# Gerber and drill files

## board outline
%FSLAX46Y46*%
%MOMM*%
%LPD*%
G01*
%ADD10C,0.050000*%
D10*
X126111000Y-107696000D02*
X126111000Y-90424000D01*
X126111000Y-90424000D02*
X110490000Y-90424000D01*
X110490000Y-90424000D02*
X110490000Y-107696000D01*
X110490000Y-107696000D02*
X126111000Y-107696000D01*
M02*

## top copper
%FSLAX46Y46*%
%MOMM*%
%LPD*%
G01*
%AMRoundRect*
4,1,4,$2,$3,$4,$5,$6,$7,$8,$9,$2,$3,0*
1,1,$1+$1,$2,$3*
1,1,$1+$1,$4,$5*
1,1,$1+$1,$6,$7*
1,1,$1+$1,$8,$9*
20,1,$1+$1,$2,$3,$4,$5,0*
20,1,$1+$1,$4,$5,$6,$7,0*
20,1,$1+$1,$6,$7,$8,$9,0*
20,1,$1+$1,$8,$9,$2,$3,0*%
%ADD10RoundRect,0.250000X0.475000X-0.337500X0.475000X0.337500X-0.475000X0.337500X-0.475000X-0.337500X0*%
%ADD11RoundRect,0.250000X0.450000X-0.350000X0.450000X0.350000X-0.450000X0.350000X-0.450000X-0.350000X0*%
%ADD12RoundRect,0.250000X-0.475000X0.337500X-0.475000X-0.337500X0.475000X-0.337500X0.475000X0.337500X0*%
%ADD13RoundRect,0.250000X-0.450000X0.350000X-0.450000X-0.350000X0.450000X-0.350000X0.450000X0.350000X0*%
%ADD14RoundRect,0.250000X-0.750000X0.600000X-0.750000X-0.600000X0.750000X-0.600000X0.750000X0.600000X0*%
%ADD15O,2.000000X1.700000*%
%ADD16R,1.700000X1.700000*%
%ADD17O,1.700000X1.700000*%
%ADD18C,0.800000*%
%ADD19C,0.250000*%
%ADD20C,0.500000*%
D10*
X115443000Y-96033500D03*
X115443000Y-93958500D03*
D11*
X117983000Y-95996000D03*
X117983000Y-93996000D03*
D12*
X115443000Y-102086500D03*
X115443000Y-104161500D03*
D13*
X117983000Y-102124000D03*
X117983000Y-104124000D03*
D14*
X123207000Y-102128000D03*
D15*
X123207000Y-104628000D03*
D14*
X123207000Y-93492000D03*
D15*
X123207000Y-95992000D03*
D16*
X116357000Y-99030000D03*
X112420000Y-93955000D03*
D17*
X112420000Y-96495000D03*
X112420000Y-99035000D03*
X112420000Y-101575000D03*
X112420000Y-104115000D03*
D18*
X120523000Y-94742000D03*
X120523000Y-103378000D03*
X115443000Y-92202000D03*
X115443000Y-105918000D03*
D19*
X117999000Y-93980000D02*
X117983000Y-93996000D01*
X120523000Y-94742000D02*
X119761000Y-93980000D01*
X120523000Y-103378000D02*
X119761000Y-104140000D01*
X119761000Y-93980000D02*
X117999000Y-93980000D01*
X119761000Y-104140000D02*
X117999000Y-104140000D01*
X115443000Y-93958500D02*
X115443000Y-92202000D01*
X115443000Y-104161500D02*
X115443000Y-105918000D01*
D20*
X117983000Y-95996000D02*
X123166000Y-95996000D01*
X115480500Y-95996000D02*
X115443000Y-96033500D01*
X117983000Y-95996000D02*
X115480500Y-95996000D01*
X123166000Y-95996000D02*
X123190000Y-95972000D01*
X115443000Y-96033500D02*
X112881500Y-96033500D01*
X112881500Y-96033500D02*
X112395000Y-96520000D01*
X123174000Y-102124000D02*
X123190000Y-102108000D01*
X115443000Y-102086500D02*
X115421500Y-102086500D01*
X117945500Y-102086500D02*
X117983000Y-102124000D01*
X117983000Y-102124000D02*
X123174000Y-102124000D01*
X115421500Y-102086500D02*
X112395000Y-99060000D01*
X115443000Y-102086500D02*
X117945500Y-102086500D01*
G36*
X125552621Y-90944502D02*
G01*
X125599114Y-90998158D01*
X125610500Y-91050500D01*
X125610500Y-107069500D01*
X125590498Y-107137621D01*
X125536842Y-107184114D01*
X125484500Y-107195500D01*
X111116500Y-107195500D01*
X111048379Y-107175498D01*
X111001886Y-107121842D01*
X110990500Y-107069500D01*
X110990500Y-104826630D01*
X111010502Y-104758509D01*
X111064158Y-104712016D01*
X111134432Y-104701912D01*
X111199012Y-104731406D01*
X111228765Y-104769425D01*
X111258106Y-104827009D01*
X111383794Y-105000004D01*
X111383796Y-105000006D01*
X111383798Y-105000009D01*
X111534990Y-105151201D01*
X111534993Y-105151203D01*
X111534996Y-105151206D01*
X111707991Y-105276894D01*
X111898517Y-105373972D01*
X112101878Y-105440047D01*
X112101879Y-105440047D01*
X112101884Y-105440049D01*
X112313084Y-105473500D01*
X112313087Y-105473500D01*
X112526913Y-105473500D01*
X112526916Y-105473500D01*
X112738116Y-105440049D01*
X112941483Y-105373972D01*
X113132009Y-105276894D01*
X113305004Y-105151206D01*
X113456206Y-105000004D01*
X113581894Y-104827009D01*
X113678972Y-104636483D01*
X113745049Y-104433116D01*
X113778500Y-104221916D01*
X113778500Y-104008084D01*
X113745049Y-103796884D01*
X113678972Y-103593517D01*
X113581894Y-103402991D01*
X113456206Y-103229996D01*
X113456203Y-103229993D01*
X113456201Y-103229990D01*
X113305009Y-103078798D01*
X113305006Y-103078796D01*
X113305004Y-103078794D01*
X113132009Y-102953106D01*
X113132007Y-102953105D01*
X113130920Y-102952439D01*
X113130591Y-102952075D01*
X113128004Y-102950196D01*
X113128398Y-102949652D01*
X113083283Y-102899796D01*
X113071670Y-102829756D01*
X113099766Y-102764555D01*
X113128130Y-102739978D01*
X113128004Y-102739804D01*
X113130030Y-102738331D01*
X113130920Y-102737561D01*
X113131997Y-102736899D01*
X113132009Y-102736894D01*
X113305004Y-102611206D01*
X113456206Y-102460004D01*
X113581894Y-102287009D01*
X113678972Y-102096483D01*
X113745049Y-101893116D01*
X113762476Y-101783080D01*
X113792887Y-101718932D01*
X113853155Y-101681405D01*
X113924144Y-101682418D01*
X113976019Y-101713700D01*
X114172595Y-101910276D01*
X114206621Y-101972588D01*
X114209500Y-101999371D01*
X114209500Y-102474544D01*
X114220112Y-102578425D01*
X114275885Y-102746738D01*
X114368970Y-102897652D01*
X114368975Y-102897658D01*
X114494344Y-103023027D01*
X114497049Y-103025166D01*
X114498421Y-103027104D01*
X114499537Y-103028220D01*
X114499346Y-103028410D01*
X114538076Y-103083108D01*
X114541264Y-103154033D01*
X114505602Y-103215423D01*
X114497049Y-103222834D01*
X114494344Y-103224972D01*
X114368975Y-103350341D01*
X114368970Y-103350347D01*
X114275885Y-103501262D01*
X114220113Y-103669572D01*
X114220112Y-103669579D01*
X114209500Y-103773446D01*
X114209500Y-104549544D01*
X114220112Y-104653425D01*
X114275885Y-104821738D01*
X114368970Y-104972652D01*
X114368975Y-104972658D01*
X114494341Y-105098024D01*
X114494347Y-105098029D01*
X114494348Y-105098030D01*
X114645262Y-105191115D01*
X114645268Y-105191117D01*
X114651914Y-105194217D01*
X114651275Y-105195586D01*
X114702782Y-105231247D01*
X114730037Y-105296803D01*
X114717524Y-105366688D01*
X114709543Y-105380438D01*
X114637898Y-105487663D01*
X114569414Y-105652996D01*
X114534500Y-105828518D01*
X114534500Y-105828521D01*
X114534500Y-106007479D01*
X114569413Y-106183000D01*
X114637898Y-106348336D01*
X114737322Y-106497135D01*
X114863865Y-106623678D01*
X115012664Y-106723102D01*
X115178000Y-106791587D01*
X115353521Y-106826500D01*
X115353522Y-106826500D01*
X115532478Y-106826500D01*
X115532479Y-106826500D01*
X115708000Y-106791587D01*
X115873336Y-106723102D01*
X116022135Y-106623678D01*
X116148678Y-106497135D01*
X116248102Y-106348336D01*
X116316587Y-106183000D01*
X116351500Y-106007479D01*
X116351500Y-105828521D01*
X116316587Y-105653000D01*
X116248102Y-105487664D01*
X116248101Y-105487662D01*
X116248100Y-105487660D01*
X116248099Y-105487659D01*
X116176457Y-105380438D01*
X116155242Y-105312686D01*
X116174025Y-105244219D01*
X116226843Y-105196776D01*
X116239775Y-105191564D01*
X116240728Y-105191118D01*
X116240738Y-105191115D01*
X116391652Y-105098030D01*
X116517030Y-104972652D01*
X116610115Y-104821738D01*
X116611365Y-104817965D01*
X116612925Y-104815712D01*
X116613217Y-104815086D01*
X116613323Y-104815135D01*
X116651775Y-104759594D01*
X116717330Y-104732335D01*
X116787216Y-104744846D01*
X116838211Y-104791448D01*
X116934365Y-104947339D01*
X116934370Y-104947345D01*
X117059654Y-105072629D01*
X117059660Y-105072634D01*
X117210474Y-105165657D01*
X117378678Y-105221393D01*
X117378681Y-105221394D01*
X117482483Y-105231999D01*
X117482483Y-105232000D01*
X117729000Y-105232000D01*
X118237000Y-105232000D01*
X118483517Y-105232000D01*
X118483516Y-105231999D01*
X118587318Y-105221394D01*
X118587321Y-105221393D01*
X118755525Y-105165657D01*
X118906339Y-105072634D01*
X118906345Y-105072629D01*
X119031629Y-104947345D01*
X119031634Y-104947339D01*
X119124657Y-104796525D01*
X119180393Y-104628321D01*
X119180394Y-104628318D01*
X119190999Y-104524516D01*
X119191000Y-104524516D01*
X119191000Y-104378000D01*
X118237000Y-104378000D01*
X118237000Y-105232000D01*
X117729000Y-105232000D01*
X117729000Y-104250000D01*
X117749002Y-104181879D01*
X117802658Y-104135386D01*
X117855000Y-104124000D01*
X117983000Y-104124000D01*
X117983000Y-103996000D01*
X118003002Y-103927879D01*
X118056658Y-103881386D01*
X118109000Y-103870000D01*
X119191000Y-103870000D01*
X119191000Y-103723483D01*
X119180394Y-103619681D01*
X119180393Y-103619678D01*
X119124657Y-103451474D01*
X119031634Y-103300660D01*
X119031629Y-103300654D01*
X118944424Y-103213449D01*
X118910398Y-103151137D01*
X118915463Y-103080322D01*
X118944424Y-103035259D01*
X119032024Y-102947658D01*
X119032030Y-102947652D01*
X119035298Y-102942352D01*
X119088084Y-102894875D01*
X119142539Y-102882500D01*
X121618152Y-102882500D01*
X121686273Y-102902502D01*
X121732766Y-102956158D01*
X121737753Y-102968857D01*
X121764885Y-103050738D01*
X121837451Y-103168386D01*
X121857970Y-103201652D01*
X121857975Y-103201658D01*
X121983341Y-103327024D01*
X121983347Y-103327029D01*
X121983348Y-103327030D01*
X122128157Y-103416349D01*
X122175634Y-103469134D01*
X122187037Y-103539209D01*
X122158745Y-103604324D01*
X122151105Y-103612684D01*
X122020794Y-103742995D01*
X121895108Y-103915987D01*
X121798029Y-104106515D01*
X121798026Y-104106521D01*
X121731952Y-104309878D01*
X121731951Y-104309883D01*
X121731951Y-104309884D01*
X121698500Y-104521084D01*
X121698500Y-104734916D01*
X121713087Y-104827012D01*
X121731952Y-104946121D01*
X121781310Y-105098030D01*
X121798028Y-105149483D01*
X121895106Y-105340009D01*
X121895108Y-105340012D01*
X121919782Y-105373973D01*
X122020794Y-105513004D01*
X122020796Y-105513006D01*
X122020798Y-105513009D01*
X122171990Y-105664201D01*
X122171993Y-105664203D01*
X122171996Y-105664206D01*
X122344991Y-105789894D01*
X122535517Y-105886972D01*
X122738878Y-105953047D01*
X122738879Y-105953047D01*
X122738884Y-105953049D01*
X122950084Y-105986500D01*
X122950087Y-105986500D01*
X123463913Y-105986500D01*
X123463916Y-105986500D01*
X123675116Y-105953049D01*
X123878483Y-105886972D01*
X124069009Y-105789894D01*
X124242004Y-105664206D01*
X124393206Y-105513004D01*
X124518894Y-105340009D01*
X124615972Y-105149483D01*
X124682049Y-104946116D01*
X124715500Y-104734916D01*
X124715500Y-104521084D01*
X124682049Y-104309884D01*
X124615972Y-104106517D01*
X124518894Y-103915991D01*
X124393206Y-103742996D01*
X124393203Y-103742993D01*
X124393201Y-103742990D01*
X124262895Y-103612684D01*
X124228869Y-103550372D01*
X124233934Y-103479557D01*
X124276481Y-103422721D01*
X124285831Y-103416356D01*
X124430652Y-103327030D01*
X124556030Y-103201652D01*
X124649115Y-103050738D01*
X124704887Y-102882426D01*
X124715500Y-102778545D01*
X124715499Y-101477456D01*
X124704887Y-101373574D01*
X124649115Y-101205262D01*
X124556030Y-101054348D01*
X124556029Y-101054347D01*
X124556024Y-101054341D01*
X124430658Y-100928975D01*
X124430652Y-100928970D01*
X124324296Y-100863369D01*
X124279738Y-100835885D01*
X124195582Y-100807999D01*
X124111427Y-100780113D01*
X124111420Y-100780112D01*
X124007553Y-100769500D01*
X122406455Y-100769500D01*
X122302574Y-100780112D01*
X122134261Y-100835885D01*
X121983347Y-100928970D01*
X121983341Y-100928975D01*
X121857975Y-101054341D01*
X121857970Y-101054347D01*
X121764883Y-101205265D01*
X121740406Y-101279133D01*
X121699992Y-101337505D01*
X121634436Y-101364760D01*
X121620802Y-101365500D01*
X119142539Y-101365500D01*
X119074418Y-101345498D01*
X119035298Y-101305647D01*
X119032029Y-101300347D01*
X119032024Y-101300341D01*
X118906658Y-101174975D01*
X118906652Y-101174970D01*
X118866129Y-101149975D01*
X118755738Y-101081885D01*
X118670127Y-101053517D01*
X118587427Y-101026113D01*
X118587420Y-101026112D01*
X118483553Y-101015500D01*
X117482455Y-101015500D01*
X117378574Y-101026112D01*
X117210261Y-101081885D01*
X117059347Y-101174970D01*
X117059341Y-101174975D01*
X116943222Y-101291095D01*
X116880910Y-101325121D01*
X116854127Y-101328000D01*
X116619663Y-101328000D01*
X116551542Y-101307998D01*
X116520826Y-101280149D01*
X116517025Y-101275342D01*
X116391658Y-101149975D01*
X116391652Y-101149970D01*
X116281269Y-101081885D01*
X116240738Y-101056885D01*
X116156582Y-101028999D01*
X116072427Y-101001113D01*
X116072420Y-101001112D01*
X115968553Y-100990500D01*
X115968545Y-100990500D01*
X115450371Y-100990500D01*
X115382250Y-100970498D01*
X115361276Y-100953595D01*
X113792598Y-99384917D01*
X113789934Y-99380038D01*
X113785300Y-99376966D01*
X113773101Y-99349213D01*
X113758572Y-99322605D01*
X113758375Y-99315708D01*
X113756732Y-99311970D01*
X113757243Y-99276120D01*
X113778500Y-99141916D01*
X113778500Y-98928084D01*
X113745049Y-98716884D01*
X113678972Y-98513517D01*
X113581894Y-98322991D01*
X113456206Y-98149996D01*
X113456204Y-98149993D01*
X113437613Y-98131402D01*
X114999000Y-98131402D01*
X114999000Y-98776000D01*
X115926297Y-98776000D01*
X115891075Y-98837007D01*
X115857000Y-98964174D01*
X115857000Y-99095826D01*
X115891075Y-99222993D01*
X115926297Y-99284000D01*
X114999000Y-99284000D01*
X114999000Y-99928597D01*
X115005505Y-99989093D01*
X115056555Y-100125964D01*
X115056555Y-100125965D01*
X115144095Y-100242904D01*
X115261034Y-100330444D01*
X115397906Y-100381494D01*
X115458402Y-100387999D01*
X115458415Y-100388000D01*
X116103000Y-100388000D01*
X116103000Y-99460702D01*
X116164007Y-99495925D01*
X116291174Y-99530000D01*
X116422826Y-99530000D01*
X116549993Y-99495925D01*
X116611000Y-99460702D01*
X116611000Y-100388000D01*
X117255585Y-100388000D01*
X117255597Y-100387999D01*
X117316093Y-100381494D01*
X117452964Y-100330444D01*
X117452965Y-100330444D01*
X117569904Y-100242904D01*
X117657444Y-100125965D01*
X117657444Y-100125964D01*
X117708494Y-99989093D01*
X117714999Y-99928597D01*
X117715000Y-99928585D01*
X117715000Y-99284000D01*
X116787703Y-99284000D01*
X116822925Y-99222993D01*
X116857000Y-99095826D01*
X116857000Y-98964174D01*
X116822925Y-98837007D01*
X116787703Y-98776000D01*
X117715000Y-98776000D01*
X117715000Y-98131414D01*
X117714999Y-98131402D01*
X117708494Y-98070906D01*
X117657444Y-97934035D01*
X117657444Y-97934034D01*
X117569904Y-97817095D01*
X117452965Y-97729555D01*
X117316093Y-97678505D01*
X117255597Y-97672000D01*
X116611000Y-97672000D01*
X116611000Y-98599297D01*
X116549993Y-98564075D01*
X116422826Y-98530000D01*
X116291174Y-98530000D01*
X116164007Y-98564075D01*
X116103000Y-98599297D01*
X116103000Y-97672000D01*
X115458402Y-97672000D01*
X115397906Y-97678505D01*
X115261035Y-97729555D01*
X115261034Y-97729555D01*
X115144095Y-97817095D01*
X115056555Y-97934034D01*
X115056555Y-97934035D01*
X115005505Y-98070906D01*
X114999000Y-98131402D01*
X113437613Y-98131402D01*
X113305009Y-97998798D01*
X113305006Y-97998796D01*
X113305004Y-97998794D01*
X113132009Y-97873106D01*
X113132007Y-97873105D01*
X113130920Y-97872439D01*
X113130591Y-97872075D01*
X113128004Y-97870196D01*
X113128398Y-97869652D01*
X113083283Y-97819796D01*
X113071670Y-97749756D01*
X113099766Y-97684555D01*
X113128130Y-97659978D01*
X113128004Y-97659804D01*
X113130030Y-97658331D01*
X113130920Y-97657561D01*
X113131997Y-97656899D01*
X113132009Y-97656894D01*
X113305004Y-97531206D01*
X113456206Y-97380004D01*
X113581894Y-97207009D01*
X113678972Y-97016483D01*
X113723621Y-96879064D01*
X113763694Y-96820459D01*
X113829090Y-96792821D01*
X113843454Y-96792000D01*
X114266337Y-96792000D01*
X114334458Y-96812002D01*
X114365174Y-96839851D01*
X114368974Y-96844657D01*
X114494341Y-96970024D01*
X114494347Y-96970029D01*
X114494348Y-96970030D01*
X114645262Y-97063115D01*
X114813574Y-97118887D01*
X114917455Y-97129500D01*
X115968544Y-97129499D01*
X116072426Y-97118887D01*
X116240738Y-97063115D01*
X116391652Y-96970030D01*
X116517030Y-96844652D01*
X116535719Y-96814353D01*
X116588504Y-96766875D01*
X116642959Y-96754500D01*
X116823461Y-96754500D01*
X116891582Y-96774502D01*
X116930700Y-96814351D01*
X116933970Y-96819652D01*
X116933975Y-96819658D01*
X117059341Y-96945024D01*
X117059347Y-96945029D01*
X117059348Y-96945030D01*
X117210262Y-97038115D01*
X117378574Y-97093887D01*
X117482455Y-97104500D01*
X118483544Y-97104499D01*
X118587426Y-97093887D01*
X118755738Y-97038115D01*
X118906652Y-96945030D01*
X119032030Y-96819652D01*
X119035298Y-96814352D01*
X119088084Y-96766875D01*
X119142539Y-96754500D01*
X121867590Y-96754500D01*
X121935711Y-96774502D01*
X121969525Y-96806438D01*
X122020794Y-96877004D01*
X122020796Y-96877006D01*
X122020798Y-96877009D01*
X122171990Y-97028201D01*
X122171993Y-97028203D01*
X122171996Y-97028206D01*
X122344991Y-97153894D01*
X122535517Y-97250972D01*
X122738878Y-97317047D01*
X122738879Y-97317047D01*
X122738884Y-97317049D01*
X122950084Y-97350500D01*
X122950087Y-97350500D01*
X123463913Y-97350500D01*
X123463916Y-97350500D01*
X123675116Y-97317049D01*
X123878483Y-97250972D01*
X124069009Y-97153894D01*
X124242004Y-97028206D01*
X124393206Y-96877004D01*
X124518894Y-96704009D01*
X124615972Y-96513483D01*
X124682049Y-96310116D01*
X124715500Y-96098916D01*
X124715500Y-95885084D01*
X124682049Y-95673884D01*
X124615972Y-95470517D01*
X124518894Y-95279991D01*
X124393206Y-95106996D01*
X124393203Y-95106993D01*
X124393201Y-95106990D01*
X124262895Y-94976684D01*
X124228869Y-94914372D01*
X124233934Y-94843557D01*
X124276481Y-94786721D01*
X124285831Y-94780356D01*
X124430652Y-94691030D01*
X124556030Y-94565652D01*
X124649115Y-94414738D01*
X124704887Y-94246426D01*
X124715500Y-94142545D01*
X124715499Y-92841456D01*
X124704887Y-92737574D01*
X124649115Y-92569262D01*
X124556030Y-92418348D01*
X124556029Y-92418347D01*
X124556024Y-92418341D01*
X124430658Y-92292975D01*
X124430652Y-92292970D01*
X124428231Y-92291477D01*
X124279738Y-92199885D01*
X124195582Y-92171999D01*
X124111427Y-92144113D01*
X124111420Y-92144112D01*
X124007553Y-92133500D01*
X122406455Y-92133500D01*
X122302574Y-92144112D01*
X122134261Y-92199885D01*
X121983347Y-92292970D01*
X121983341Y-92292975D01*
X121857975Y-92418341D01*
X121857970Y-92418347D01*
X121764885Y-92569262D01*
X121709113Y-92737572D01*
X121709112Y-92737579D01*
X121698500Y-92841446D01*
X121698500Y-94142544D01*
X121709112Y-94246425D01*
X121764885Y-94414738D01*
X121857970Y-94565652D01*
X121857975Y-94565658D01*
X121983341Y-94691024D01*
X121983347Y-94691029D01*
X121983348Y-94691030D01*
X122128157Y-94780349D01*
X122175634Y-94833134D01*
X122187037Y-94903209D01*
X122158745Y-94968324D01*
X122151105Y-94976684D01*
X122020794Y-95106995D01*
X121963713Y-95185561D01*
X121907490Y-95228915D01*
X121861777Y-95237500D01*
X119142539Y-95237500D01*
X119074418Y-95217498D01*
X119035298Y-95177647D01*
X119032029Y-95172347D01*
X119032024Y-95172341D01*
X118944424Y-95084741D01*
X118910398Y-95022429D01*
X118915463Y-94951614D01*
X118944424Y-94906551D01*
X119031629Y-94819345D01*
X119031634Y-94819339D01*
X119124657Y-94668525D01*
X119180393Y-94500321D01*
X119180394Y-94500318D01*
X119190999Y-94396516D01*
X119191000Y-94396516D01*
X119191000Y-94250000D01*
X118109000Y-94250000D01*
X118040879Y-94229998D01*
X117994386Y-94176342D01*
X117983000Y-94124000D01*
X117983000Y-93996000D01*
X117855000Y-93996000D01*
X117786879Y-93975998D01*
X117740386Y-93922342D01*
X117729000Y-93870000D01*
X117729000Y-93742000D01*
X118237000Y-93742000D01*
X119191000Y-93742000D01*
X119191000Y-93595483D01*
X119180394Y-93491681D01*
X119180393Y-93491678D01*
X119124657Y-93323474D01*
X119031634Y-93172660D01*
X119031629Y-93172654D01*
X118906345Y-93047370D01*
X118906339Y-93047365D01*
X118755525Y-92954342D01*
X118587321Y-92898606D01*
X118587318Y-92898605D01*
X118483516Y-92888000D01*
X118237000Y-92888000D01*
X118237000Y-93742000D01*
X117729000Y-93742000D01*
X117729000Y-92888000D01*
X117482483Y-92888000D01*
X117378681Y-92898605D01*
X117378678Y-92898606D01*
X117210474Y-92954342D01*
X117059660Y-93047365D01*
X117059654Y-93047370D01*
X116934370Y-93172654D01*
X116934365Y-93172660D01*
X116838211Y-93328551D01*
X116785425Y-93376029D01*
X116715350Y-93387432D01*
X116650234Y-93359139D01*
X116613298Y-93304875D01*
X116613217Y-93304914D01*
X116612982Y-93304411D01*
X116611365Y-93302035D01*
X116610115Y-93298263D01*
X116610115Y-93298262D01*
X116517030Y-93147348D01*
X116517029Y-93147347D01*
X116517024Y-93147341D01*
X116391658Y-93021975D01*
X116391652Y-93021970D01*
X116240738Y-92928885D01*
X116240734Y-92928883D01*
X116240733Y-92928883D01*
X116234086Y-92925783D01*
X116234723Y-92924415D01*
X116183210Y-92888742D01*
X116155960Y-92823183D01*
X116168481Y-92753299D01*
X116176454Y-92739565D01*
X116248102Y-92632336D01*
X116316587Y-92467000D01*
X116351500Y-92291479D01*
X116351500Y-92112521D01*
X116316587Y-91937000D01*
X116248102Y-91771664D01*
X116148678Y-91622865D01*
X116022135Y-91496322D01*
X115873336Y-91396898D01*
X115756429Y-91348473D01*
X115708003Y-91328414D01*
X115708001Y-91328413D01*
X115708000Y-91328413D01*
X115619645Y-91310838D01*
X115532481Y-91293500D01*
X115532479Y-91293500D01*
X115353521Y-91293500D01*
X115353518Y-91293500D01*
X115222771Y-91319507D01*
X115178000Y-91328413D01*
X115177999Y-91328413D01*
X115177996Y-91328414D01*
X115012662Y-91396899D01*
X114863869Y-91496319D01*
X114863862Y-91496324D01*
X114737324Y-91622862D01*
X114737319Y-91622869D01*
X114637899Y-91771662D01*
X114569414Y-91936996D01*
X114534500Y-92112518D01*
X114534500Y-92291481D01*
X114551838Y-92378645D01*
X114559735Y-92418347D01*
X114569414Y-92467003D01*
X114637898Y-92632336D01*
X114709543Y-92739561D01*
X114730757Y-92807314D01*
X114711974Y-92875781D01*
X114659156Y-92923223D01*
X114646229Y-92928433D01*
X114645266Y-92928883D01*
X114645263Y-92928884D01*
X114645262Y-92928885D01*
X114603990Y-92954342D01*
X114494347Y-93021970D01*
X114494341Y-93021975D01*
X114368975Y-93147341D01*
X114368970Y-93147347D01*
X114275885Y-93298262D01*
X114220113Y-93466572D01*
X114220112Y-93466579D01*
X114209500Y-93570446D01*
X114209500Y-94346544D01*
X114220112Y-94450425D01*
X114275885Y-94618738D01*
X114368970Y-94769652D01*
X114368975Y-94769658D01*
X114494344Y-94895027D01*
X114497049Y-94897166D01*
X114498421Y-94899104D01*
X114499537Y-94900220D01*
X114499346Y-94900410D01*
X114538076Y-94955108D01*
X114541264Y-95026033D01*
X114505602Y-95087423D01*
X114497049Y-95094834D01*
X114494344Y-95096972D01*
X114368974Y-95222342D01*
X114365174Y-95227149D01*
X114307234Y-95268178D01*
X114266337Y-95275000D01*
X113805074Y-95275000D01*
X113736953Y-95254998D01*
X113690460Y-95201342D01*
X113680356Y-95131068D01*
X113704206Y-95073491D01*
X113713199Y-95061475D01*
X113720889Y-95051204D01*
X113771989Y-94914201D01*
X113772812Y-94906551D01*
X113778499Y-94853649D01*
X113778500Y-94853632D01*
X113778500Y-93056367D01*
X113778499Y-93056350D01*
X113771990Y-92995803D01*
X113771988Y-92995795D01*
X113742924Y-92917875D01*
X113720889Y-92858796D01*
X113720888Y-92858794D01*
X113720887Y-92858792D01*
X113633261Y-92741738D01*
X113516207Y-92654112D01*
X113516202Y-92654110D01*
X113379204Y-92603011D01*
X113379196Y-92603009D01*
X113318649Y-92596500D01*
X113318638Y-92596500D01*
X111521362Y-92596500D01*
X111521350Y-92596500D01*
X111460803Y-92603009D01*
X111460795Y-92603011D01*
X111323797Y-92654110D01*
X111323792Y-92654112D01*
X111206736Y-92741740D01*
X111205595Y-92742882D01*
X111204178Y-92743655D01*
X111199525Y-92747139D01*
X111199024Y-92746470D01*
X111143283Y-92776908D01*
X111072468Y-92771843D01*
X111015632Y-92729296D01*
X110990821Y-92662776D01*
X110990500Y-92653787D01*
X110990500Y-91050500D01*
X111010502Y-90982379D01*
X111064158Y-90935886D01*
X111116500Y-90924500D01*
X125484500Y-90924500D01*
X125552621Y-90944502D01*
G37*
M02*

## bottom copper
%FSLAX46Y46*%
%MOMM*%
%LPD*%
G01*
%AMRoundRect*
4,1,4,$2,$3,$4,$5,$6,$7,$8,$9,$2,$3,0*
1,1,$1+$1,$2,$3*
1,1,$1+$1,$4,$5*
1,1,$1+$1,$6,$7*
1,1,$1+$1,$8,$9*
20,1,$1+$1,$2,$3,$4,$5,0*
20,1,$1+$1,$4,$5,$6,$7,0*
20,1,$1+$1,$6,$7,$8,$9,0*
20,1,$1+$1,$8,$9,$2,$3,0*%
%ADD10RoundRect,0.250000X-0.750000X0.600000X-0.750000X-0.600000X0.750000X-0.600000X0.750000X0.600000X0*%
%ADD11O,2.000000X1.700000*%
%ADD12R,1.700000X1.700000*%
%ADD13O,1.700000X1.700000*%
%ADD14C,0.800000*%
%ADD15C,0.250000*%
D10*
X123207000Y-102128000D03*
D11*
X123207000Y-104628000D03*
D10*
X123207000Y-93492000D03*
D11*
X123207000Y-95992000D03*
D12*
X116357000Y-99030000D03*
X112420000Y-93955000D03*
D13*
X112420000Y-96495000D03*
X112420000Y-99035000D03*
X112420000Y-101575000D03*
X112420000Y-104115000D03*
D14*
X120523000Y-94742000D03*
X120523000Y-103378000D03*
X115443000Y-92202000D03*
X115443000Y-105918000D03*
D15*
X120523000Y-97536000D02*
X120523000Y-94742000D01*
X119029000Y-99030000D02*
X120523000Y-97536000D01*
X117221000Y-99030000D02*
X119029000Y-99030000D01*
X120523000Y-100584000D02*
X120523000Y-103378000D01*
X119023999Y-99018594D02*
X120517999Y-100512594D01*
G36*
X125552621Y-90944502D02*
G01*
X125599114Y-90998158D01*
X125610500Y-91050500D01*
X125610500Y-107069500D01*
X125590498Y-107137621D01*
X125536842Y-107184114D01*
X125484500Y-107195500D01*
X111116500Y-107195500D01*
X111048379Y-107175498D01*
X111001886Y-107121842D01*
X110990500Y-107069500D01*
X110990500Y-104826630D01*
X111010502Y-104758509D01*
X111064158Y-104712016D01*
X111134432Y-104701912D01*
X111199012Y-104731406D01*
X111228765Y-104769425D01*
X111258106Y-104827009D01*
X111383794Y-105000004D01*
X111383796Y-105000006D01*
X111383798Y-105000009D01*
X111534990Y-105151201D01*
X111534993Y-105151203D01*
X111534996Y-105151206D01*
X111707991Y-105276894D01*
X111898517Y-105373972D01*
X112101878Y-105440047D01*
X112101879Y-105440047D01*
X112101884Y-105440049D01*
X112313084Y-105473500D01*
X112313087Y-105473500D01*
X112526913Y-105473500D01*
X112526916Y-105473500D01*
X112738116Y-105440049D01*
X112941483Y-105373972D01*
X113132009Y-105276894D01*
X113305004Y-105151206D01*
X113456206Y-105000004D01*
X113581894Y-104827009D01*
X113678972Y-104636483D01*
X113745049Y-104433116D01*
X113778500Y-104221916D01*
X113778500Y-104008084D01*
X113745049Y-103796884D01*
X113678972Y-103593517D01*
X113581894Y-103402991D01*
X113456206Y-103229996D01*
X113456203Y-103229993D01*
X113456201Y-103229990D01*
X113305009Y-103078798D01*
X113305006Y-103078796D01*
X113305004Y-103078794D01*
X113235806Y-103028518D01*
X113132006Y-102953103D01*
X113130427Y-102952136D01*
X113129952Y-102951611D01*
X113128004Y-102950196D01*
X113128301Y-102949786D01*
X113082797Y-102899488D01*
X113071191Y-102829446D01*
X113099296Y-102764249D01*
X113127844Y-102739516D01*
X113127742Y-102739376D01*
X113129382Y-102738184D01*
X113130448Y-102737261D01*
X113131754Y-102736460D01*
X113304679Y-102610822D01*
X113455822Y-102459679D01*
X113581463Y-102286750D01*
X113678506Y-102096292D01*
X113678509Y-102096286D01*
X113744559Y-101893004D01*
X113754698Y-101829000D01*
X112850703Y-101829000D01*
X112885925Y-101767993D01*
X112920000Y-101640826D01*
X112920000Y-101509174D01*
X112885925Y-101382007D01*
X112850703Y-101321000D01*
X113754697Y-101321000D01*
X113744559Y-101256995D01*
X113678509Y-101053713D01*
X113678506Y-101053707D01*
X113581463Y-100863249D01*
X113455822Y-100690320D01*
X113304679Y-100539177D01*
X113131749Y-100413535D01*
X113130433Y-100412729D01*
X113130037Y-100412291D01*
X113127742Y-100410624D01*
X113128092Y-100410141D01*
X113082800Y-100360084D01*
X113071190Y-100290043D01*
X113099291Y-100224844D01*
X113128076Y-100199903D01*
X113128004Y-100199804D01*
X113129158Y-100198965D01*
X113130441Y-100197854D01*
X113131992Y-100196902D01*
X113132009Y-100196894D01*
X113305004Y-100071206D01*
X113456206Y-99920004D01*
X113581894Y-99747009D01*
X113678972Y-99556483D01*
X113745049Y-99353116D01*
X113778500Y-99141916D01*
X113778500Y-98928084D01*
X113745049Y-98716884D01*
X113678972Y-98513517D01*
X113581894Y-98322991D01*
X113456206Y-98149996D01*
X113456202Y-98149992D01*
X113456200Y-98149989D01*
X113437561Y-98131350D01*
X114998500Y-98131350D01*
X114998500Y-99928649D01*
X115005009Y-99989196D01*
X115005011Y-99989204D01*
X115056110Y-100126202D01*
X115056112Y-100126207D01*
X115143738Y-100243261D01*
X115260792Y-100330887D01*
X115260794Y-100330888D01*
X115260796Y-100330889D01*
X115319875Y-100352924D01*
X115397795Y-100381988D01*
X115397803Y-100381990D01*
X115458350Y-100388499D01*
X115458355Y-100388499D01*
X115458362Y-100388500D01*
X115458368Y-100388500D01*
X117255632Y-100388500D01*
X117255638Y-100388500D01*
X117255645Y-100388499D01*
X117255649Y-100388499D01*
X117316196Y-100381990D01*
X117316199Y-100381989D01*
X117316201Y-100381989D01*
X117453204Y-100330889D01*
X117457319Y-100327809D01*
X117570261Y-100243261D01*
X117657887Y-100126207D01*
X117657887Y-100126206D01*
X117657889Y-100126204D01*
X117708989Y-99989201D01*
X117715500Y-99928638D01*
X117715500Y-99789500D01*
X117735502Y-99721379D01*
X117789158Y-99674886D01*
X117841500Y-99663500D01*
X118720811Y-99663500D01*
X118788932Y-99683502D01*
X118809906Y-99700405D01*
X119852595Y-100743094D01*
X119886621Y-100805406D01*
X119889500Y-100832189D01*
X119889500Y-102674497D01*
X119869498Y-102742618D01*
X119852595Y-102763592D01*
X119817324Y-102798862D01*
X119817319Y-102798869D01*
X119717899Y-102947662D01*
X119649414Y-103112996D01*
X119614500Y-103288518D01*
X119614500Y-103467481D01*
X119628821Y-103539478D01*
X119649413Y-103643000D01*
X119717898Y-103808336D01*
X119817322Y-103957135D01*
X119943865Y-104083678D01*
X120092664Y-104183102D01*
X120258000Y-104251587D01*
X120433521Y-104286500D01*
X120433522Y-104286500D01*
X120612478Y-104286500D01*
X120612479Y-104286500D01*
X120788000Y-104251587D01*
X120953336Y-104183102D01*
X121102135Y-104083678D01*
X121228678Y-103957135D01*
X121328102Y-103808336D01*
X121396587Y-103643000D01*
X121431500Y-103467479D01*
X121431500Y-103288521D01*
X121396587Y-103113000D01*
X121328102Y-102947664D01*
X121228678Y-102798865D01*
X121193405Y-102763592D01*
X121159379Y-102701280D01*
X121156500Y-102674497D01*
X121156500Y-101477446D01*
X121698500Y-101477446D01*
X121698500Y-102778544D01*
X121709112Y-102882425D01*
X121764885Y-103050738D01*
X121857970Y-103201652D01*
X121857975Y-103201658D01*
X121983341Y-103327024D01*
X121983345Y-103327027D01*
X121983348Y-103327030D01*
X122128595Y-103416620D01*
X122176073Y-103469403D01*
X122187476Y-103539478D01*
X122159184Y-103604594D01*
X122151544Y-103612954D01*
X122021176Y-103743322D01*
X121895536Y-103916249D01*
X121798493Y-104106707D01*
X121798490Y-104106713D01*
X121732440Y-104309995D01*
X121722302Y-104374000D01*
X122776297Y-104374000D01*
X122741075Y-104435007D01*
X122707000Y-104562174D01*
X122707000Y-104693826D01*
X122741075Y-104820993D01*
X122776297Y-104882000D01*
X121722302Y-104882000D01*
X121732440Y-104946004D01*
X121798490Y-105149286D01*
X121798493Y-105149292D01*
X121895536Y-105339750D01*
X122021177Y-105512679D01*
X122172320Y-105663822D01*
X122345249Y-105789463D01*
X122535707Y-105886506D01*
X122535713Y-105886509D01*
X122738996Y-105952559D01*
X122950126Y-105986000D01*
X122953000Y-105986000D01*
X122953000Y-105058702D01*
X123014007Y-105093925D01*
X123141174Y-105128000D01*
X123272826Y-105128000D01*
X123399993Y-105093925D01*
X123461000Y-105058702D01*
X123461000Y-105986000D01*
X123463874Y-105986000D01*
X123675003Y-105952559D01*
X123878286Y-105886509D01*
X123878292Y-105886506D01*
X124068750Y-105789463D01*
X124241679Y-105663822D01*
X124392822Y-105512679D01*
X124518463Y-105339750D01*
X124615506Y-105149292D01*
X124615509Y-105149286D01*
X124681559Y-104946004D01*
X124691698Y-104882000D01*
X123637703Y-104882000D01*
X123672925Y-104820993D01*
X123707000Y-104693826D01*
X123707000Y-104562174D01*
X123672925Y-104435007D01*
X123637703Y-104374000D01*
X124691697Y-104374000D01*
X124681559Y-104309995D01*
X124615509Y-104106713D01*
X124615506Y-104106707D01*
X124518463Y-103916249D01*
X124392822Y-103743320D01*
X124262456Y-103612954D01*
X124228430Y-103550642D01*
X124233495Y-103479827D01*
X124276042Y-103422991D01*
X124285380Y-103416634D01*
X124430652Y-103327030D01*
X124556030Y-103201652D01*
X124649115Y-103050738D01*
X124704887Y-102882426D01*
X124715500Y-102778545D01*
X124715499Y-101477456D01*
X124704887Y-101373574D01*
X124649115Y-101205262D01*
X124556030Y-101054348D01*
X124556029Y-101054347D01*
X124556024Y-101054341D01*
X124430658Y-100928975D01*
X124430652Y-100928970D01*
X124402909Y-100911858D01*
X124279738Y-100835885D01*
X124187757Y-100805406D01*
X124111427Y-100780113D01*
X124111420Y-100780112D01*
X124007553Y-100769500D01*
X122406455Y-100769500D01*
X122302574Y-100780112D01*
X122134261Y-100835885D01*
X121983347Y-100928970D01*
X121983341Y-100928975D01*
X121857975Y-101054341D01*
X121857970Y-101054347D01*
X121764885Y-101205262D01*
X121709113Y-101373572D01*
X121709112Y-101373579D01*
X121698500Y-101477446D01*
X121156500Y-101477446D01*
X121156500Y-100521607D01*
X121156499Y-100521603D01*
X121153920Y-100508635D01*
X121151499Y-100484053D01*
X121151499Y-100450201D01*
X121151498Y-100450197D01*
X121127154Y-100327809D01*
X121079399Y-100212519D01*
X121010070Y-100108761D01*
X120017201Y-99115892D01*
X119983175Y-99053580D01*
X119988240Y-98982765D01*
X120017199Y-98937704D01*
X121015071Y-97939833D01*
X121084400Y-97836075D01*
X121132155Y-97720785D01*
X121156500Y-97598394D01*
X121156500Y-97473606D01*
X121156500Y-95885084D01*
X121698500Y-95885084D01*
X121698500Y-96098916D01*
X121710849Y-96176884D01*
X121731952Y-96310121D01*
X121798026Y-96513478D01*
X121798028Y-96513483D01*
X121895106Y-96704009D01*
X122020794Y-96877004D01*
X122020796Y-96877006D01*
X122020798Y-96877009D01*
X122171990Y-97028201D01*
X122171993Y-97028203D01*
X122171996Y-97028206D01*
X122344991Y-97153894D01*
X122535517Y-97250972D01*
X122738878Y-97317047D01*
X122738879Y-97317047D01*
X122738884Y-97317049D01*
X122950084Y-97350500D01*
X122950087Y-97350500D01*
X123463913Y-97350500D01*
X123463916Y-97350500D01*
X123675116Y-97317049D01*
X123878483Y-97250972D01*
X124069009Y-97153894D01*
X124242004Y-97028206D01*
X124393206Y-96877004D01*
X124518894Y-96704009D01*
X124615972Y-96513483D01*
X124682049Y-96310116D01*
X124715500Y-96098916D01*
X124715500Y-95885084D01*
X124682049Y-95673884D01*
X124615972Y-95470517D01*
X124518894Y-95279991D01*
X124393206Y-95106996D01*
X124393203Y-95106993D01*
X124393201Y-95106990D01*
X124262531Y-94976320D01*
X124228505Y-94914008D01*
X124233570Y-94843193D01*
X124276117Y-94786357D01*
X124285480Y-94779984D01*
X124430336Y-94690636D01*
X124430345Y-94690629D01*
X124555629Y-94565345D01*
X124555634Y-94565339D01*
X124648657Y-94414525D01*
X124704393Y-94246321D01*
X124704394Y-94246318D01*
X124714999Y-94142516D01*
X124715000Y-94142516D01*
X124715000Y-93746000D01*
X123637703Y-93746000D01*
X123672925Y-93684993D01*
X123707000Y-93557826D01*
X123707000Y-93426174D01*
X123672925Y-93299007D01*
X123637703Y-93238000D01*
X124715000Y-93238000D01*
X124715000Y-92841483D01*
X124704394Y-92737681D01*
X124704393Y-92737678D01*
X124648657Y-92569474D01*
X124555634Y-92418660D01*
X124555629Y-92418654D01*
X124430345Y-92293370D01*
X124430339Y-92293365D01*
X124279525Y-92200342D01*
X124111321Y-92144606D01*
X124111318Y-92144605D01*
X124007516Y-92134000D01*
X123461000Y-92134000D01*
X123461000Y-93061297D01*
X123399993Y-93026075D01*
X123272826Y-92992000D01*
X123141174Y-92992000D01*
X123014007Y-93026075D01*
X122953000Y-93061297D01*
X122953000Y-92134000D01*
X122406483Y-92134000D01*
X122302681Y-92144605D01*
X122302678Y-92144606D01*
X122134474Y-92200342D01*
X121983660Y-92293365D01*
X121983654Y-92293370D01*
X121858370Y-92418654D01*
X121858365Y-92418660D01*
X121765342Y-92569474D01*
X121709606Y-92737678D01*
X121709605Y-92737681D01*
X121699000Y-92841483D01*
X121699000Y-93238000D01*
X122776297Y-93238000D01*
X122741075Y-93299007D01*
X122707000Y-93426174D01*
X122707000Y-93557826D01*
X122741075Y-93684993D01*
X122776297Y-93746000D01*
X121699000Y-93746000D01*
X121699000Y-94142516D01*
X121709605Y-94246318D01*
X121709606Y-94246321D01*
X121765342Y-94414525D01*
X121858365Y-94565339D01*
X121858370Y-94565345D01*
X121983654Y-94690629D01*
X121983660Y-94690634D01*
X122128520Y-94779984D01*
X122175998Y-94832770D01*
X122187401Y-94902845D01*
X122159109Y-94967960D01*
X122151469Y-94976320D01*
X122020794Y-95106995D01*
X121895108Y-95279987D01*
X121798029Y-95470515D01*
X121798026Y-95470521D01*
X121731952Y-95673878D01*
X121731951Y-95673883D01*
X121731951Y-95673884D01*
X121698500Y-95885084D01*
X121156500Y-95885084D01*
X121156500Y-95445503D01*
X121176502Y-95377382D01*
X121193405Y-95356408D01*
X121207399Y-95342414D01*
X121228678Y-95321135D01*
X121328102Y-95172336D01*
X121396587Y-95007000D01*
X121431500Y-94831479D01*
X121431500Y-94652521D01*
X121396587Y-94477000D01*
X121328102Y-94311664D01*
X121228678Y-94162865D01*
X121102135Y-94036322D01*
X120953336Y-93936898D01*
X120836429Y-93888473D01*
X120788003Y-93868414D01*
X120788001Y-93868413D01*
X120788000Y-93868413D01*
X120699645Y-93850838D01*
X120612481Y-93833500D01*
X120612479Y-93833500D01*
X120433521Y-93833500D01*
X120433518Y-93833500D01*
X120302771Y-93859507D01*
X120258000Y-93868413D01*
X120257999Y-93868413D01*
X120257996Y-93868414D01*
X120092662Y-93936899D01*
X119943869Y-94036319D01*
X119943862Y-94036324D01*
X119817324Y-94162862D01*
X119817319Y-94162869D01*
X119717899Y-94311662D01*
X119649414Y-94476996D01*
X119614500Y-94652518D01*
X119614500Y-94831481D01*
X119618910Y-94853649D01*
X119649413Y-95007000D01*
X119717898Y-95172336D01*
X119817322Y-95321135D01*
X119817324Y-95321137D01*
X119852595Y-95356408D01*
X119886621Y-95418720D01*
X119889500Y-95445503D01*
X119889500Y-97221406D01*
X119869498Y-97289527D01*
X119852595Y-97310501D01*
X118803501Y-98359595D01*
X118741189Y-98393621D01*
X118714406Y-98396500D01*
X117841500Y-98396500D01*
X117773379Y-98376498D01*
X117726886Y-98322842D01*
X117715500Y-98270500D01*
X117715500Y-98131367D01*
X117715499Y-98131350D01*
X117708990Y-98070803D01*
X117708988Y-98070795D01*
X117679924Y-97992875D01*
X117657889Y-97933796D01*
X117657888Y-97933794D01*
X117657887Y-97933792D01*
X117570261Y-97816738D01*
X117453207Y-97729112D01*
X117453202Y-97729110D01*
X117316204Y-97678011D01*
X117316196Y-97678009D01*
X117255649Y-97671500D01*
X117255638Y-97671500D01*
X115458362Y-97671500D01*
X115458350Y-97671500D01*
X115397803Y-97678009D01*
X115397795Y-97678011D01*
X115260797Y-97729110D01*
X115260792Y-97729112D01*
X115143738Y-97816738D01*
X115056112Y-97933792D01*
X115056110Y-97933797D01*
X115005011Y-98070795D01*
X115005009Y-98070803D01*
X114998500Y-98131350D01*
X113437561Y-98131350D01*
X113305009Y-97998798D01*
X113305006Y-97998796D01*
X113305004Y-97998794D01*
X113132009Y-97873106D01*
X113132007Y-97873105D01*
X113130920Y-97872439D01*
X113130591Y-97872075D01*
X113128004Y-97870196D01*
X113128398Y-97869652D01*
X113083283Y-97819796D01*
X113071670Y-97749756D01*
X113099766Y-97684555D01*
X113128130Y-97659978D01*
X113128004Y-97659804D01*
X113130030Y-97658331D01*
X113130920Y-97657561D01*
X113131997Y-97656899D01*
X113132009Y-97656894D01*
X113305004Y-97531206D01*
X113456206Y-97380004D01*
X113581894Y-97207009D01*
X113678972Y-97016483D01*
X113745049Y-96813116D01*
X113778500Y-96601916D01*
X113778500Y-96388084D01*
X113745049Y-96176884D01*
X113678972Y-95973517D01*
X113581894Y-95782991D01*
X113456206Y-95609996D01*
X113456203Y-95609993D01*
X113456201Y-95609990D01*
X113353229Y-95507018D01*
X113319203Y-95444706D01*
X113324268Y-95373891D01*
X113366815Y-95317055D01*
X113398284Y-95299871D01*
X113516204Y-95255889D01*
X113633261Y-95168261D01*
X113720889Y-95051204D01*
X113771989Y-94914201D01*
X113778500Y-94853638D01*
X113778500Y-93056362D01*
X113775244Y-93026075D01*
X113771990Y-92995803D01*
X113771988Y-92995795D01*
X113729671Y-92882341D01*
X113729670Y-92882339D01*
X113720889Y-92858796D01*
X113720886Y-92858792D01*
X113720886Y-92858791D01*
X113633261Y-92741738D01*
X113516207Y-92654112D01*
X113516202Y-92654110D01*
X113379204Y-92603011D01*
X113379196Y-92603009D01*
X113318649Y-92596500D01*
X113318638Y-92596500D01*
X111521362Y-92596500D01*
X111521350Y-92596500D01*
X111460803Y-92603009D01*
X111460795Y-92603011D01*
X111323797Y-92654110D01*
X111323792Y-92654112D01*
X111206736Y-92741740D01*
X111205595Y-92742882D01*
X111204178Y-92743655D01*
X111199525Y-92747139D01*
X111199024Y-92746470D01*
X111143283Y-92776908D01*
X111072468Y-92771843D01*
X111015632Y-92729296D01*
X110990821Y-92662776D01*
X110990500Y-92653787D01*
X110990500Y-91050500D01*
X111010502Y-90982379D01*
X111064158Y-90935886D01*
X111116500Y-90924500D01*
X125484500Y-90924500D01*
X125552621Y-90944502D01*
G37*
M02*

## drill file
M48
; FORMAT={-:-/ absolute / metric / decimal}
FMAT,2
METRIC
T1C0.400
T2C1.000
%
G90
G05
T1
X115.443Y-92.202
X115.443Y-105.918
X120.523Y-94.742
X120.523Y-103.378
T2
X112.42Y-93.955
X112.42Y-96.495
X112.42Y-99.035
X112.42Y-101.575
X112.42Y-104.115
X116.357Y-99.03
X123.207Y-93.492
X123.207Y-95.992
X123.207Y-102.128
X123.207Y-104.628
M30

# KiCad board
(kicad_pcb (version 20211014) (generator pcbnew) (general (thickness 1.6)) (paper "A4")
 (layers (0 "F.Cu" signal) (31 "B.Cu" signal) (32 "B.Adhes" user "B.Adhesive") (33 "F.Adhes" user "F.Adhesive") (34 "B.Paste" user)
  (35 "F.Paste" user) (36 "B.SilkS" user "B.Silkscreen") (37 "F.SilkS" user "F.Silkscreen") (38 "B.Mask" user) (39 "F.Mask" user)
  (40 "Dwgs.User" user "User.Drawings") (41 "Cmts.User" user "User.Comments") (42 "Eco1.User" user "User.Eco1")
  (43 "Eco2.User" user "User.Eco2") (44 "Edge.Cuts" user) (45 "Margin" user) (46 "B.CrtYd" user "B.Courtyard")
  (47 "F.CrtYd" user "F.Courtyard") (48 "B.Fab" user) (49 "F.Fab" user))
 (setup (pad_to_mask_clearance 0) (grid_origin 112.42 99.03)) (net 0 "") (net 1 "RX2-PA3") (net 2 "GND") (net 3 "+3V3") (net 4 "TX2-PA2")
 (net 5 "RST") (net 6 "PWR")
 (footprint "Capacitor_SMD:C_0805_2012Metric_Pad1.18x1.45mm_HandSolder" (layer "F.Cu") (at 115.443 94.996 90)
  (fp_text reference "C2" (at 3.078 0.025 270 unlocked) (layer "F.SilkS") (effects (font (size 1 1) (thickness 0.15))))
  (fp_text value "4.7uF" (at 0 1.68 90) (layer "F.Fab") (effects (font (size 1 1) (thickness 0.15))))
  (pad "1" smd roundrect locked (at -1.0375 0 90) (size 1.175 1.45) (layers "F.Cu" "F.Paste" "F.Mask") (roundrect_rratio 0.2127659574)
   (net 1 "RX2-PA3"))
  (pad "2" smd roundrect locked (at 1.0375 0 90) (size 1.175 1.45) (layers "F.Cu" "F.Paste" "F.Mask") (roundrect_rratio 0.2127659574)
   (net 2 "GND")))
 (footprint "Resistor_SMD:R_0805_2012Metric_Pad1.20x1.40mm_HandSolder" (layer "F.Cu") (at 117.983 94.996 90)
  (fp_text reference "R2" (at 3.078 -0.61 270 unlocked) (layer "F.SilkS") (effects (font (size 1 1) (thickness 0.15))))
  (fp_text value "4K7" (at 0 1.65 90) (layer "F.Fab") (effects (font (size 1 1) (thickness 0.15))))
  (pad "1" smd roundrect locked (at -1 0 90) (size 1.2 1.4) (layers "F.Cu" "F.Paste" "F.Mask") (roundrect_rratio 0.2083333333)
   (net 1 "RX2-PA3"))
  (pad "2" smd roundrect locked (at 1 0 90) (size 1.2 1.4) (layers "F.Cu" "F.Paste" "F.Mask") (roundrect_rratio 0.2083333333) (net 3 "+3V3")))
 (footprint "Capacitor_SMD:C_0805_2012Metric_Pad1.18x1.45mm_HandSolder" (layer "F.Cu") (at 115.443 103.124 -90)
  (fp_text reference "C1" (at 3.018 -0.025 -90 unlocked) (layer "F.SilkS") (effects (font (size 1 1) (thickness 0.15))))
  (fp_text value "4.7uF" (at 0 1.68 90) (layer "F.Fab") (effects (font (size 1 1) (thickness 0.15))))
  (pad "1" smd roundrect locked (at -1.0375 0 270) (size 1.175 1.45) (layers "F.Cu" "F.Paste" "F.Mask") (roundrect_rratio 0.2127659574)
   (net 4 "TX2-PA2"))
  (pad "2" smd roundrect locked (at 1.0375 0 270) (size 1.175 1.45) (layers "F.Cu" "F.Paste" "F.Mask") (roundrect_rratio 0.2127659574)
   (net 2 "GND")))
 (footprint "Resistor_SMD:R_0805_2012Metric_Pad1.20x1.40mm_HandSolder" (layer "F.Cu") (at 117.983 103.124 -90)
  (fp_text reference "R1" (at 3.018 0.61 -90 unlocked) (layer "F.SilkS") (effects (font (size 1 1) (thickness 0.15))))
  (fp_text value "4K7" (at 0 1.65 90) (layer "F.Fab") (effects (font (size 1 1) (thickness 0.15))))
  (pad "1" smd roundrect locked (at -1 0 270) (size 1.2 1.4) (layers "F.Cu" "F.Paste" "F.Mask") (roundrect_rratio 0.2083333333)
   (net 4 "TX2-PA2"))
  (pad "2" smd roundrect locked (at 1 0 270) (size 1.2 1.4) (layers "F.Cu" "F.Paste" "F.Mask") (roundrect_rratio 0.2083333333)
   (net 3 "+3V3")))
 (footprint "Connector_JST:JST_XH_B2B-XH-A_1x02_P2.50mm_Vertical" (layer "F.Cu") (at 123.207 102.128 -90)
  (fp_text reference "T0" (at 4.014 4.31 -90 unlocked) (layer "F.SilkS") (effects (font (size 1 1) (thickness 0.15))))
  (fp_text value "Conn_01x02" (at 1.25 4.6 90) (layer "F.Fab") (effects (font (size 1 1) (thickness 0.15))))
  (pad "1" thru_hole roundrect locked (at 0 0 270) (size 1.7 2) (drill 1) (layers *.Cu *.Mask) (roundrect_rratio 0.1470588235)
   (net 4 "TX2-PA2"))
  (pad "2" thru_hole oval locked (at 2.5 0 270) (size 1.7 2) (drill 1) (layers *.Cu *.Mask) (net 2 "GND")))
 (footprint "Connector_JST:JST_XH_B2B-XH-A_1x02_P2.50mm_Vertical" (layer "F.Cu") (at 123.207 93.492 -90)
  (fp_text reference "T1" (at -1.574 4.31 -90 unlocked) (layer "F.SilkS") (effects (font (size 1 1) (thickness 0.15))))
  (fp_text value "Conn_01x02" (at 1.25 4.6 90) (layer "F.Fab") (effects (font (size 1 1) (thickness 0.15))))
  (pad "1" thru_hole roundrect locked (at 0 0 270) (size 1.7 2) (drill 1) (layers *.Cu *.Mask) (roundrect_rratio 0.1470588235) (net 2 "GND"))
  (pad "2" thru_hole oval locked (at 2.5 0 270) (size 1.7 2) (drill 1) (layers *.Cu *.Mask) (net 1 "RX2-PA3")))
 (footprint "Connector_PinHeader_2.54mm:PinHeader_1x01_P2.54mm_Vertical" (layer "F.Cu") (at 116.357 99.03)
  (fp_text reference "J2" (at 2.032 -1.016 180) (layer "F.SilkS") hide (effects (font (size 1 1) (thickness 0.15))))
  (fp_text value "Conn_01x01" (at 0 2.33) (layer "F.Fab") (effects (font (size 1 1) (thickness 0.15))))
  (pad "1" thru_hole rect locked (at 0 0) (size 1.7 1.7) (drill 1) (layers *.Cu *.Mask) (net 3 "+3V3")))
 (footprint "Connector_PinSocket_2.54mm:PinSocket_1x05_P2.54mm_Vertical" (layer "B.Cu") (at 112.42 93.955 180)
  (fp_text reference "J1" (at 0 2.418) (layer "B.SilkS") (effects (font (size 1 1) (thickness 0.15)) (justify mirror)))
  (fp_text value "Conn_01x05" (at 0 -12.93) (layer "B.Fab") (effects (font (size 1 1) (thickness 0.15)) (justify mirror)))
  (pad "1" thru_hole rect locked (at 0 0 180) (size 1.7 1.7) (drill 1) (layers *.Cu *.Mask) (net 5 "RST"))
  (pad "2" thru_hole oval locked (at 0 -2.54 180) (size 1.7 1.7) (drill 1) (layers *.Cu *.Mask) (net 1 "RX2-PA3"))
  (pad "3" thru_hole oval locked (at 0 -5.08 180) (size 1.7 1.7) (drill 1) (layers *.Cu *.Mask) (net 4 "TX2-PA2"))
  (pad "4" thru_hole oval locked (at 0 -7.62 180) (size 1.7 1.7) (drill 1) (layers *.Cu *.Mask) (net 2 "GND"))
  (pad "5" thru_hole oval locked (at 0 -10.16 180) (size 1.7 1.7) (drill 1) (layers *.Cu *.Mask) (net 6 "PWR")))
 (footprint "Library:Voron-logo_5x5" (layer "B.Cu") (at 115.976 93.442 -90)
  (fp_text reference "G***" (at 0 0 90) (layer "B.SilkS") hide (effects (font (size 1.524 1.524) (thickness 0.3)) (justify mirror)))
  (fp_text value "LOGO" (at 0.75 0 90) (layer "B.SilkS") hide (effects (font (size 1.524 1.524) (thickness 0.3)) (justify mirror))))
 (gr_line (start 126.111 107.696) (end 126.111 90.424) (layer "Edge.Cuts") (width 0.05))
 (gr_line (start 126.111 90.424) (end 110.49 90.424) (layer "Edge.Cuts") (width 0.05))
 (gr_line (start 110.49 90.424) (end 110.49 107.696) (layer "Edge.Cuts") (width 0.05))
 (gr_line (start 110.49 107.696) (end 126.111 107.696) (layer "Edge.Cuts") (width 0.05))
 (segment (start 117.999 93.98) (end 117.983 93.996) (width 0.25) (layer "F.Cu") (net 3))
 (segment (start 120.523 94.742) (end 119.761 93.98) (width 0.25) (layer "F.Cu") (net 3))
 (segment (start 120.523 103.378) (end 119.761 104.14) (width 0.25) (layer "F.Cu") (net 3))
 (segment (start 119.761 93.98) (end 117.999 93.98) (width 0.25) (layer "F.Cu") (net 3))
 (segment (start 119.761 104.14) (end 117.999 104.14) (width 0.25) (layer "F.Cu") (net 3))
 (via (at 120.523 94.742) (size 0.8) (drill 0.4) (layers "F.Cu" "B.Cu") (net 3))
 (via (at 120.523 103.378) (size 0.8) (drill 0.4) (layers "F.Cu" "B.Cu") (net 3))
 (segment (start 120.523 97.536) (end 120.523 94.742) (width 0.25) (layer "B.Cu") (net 3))
 (segment (start 119.029 99.03) (end 120.523 97.536) (width 0.25) (layer "B.Cu") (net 3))
 (segment (start 117.221 99.03) (end 119.029 99.03) (width 0.25) (layer "B.Cu") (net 3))
 (segment (start 120.523 100.584) (end 120.523 103.378) (width 0.25) (layer "B.Cu") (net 3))
 (segment (start 119.023999 99.018594) (end 120.517999 100.512594) (width 0.25) (layer "B.Cu") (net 3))
 (segment (start 115.443 93.9585) (end 115.443 92.202) (width 0.25) (layer "F.Cu") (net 2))
 (segment (start 115.443 104.1615) (end 115.443 105.918) (width 0.25) (layer "F.Cu") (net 2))
 (via (at 115.443 92.202) (size 0.8) (drill 0.4) (layers "F.Cu" "B.Cu") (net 2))
 (via (at 115.443 105.918) (size 0.8) (drill 0.4) (layers "F.Cu" "B.Cu") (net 2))
 (segment (start 117.983 95.996) (end 123.166 95.996) (width 0.5) (layer "F.Cu") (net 1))
 (segment (start 115.4805 95.996) (end 115.443 96.0335) (width 0.5) (layer "F.Cu") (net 1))
 (segment (start 117.983 95.996) (end 115.4805 95.996) (width 0.5) (layer "F.Cu") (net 1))
 (segment (start 123.166 95.996) (end 123.19 95.972) (width 0.5) (layer "F.Cu") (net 1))
 (segment (start 115.443 96.0335) (end 112.8815 96.0335) (width 0.5) (layer "F.Cu") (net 1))
 (segment (start 112.8815 96.0335) (end 112.395 96.52) (width 0.5) (layer "F.Cu") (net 1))
 (segment (start 123.174 102.124) (end 123.19 102.108) (width 0.5) (layer "F.Cu") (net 4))
 (segment (start 115.443 102.0865) (end 115.4215 102.0865) (width 0.5) (layer "F.Cu") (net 4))
 (segment (start 117.9455 102.0865) (end 117.983 102.124) (width 0.5) (layer "F.Cu") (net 4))
 (segment (start 117.983 102.124) (end 123.174 102.124) (width 0.5) (layer "F.Cu") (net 4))
 (segment (start 115.4215 102.0865) (end 112.395 99.06) (width 0.5) (layer "F.Cu") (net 4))
 (segment (start 115.443 102.0865) (end 117.9455 102.0865) (width 0.5) (layer "F.Cu") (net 4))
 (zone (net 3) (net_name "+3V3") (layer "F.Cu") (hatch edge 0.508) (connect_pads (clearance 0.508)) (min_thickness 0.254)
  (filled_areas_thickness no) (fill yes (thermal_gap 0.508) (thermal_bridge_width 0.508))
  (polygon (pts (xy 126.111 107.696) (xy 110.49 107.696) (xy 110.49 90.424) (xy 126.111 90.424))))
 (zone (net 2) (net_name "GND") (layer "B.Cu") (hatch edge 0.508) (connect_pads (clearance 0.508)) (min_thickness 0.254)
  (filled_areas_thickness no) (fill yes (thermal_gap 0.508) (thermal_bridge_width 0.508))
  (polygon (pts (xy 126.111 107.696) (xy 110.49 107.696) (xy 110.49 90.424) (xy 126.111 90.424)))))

